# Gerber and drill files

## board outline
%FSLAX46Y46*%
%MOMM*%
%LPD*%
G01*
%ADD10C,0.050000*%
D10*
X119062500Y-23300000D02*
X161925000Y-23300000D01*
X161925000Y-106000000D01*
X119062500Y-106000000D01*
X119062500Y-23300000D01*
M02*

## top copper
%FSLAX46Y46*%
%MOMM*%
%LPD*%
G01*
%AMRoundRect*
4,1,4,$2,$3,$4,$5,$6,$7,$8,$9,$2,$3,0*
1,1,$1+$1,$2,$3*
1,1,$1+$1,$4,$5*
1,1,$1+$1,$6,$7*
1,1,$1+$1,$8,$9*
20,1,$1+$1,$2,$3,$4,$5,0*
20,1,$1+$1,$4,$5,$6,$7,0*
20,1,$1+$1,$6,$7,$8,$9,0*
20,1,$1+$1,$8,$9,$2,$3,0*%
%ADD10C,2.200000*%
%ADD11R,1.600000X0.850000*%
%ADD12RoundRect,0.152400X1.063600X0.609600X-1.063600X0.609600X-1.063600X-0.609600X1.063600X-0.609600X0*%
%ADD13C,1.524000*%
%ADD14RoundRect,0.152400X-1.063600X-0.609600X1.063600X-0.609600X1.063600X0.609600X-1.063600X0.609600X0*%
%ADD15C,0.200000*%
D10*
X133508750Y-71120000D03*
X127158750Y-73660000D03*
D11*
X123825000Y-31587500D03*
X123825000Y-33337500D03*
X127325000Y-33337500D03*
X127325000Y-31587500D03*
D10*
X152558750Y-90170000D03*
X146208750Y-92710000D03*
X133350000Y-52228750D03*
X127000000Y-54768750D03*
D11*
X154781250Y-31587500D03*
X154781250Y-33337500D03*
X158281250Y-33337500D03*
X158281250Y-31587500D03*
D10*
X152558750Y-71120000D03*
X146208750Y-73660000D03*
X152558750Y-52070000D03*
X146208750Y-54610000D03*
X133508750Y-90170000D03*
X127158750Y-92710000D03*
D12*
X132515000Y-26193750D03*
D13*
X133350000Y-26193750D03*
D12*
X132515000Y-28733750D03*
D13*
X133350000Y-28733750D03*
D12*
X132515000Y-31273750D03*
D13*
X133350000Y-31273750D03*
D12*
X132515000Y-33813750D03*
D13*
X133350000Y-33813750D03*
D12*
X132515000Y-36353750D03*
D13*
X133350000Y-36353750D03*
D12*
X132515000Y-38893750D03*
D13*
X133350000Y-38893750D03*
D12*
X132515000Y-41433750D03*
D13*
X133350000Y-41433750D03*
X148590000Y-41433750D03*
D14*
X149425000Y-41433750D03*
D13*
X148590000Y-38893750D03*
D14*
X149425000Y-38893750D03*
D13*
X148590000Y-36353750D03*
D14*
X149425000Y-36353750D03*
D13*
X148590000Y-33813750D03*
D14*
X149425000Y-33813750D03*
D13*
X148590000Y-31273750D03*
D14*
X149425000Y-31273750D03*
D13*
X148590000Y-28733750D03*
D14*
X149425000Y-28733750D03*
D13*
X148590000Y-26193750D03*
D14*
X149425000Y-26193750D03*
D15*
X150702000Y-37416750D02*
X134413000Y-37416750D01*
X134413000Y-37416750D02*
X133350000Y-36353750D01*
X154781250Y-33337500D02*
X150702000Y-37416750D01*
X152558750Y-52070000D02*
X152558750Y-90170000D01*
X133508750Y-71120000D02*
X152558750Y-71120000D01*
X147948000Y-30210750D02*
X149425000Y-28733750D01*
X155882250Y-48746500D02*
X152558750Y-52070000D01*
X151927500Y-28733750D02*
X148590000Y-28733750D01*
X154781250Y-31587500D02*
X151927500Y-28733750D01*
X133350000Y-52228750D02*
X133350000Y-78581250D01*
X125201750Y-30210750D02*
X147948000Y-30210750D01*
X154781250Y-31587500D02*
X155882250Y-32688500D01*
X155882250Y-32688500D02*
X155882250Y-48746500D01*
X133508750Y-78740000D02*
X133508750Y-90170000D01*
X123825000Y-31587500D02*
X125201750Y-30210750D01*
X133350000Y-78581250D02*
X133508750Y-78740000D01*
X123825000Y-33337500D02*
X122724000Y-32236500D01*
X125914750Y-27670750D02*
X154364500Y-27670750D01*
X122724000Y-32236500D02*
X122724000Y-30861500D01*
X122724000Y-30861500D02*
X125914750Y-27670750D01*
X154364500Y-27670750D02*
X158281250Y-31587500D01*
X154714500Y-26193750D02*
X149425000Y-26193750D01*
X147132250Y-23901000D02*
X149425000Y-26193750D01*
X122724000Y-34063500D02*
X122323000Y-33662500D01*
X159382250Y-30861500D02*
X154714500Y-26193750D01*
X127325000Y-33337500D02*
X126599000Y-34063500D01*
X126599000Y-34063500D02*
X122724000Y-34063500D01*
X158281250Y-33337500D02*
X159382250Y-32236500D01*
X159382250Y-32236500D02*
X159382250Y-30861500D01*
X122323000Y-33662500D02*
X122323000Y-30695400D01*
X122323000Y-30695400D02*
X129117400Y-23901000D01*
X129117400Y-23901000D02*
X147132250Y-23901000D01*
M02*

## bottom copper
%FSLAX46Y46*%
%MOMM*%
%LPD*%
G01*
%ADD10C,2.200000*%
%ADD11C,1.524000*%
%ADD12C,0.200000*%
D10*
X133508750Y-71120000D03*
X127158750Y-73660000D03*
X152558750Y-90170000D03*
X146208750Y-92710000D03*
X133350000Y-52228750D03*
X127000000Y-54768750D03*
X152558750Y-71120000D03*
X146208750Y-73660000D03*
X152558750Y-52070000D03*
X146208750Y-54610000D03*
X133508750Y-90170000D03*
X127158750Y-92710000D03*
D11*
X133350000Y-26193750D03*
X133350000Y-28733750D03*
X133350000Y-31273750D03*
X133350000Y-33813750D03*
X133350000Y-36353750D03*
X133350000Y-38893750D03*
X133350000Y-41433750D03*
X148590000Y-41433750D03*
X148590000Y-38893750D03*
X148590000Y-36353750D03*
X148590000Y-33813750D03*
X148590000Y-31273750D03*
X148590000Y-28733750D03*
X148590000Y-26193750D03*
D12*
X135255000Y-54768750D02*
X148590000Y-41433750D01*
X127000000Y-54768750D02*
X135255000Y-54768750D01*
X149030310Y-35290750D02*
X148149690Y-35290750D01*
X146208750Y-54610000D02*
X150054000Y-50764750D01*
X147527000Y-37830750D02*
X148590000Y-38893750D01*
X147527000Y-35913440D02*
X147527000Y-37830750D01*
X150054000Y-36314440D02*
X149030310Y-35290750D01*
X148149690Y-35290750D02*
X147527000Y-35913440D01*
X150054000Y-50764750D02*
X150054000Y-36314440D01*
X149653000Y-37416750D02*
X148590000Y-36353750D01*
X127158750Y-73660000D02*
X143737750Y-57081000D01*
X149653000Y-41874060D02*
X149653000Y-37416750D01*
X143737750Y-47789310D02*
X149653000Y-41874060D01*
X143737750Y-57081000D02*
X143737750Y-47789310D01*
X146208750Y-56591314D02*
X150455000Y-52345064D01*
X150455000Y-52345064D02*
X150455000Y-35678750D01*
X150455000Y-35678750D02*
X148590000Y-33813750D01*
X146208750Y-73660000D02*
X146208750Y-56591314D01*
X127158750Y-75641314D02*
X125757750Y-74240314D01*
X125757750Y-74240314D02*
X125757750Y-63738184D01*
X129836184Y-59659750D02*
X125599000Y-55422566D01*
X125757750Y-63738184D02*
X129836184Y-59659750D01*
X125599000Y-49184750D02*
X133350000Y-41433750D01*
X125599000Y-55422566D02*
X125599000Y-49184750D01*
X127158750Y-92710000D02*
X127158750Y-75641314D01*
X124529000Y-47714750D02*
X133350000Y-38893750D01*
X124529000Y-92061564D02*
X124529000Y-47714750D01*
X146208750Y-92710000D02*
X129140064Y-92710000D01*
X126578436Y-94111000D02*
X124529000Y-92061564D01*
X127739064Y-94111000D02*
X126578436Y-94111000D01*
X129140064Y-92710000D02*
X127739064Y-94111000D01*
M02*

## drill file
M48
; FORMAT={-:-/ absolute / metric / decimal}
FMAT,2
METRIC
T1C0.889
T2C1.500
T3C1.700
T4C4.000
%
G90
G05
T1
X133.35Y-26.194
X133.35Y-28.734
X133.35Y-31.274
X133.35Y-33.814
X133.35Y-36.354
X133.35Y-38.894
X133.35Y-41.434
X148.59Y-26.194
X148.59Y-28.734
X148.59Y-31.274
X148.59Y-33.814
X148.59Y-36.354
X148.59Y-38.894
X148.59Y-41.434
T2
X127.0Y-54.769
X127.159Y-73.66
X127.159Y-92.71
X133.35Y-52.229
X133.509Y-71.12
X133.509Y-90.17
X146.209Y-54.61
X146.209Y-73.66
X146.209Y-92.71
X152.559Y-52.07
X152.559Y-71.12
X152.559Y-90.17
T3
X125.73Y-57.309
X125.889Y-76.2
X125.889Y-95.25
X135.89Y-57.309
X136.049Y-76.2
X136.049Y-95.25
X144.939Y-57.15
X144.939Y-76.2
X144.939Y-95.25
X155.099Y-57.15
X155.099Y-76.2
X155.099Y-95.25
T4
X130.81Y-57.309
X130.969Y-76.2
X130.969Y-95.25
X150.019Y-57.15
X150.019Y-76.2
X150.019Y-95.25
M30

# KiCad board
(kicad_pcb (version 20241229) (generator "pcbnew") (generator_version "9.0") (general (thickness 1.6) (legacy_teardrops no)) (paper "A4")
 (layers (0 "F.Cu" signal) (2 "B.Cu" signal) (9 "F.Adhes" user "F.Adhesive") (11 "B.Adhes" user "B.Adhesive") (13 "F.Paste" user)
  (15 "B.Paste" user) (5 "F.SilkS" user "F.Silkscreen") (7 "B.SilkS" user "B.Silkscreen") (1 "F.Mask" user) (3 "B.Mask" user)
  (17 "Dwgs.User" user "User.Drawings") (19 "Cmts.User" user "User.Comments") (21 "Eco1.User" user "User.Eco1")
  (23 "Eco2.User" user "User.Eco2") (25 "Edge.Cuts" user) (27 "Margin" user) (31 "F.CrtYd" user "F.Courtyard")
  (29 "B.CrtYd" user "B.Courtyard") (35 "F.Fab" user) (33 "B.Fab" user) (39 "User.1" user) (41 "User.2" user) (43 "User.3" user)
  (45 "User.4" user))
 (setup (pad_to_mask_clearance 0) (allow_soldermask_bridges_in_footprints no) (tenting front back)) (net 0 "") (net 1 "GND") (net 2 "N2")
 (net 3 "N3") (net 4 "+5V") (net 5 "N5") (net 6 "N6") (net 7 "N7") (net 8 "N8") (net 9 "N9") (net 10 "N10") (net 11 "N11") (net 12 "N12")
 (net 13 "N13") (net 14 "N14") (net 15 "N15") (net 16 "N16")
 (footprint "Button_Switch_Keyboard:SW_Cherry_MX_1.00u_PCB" (layer "F.Cu") (at 133.50875 71.12)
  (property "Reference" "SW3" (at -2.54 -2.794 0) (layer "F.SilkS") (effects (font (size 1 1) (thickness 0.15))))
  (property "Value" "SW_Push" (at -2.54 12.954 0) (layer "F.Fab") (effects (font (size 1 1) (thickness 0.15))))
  (pad "" np_thru_hole circle (at -7.62 5.08) (size 1.7 1.7) (drill 1.7) (layers "*.Cu" "*.Mask"))
  (pad "" np_thru_hole circle (at -2.54 5.08) (size 4 4) (drill 4) (layers "*.Cu" "*.Mask"))
  (pad "" np_thru_hole circle (at 2.54 5.08) (size 1.7 1.7) (drill 1.7) (layers "*.Cu" "*.Mask"))
  (pad "1" thru_hole circle (at 0 0) (size 2.2 2.2) (drill 1.5) (layers "*.Cu" "*.Mask") (remove_unused_layers no) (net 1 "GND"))
  (pad "2" thru_hole circle (at -6.35 2.54) (size 2.2 2.2) (drill 1.5) (layers "*.Cu" "*.Mask") (remove_unused_layers no) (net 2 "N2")))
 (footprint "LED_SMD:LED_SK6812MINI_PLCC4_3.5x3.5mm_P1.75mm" (layer "F.Cu") (at 125.575 32.4625)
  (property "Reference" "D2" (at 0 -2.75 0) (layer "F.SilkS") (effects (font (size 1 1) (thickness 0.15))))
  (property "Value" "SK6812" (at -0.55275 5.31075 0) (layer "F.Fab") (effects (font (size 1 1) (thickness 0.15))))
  (pad "1" smd rect (at -1.75 -0.875) (size 1.6 0.85) (layers "F.Cu" "F.Mask" "F.Paste") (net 1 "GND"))
  (pad "2" smd rect (at -1.75 0.875) (size 1.6 0.85) (layers "F.Cu" "F.Mask" "F.Paste") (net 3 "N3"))
  (pad "3" smd rect (at 1.75 0.875) (size 1.6 0.85) (layers "F.Cu" "F.Mask" "F.Paste") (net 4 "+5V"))
  (pad "4" smd rect (at 1.75 -0.875) (size 1.6 0.85) (layers "F.Cu" "F.Mask" "F.Paste") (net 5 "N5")))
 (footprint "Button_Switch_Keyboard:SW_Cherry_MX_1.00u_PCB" (layer "F.Cu") (at 152.55875 90.17)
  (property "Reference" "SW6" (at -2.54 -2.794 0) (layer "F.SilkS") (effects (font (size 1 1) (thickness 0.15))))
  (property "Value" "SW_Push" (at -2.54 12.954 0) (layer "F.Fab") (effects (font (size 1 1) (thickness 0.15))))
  (pad "" np_thru_hole circle (at -7.62 5.08) (size 1.7 1.7) (drill 1.7) (layers "*.Cu" "*.Mask"))
  (pad "" np_thru_hole circle (at -2.54 5.08) (size 4 4) (drill 4) (layers "*.Cu" "*.Mask"))
  (pad "" np_thru_hole circle (at 2.54 5.08) (size 1.7 1.7) (drill 1.7) (layers "*.Cu" "*.Mask"))
  (pad "1" thru_hole circle (at 0 0) (size 2.2 2.2) (drill 1.5) (layers "*.Cu" "*.Mask") (remove_unused_layers no) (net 1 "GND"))
  (pad "2" thru_hole circle (at -6.35 2.54) (size 2.2 2.2) (drill 1.5) (layers "*.Cu" "*.Mask") (remove_unused_layers no) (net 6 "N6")))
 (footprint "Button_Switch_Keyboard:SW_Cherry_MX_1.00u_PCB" (layer "F.Cu") (at 133.35 52.22875)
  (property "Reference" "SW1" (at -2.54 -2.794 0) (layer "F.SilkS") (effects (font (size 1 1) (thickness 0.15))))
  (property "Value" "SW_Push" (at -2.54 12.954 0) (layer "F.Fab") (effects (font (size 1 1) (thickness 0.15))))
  (pad "" np_thru_hole circle (at -7.62 5.08) (size 1.7 1.7) (drill 1.7) (layers "*.Cu" "*.Mask"))
  (pad "" np_thru_hole circle (at -2.54 5.08) (size 4 4) (drill 4) (layers "*.Cu" "*.Mask"))
  (pad "" np_thru_hole circle (at 2.54 5.08) (size 1.7 1.7) (drill 1.7) (layers "*.Cu" "*.Mask"))
  (pad "1" thru_hole circle (at 0 0) (size 2.2 2.2) (drill 1.5) (layers "*.Cu" "*.Mask") (remove_unused_layers no) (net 1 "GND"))
  (pad "2" thru_hole circle (at -6.35 2.54) (size 2.2 2.2) (drill 1.5) (layers "*.Cu" "*.Mask") (remove_unused_layers no) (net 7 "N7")))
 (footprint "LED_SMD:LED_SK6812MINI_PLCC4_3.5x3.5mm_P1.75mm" (layer "F.Cu") (at 156.53125 32.4625)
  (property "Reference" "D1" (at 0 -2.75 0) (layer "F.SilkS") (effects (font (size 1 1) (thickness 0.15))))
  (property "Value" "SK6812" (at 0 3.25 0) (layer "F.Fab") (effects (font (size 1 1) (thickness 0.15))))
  (pad "1" smd rect (at -1.75 -0.875) (size 1.6 0.85) (layers "F.Cu" "F.Mask" "F.Paste") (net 1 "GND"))
  (pad "2" smd rect (at -1.75 0.875) (size 1.6 0.85) (layers "F.Cu" "F.Mask" "F.Paste") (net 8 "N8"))
  (pad "3" smd rect (at 1.75 0.875) (size 1.6 0.85) (layers "F.Cu" "F.Mask" "F.Paste") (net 4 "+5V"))
  (pad "4" smd rect (at 1.75 -0.875) (size 1.6 0.85) (layers "F.Cu" "F.Mask" "F.Paste") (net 3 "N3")))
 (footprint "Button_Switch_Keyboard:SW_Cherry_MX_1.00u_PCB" (layer "F.Cu") (at 152.55875 71.12)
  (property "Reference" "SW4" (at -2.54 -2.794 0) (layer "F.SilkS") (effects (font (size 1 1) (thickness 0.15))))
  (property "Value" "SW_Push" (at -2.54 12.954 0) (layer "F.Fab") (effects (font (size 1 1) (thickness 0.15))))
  (pad "" np_thru_hole circle (at -7.62 5.08) (size 1.7 1.7) (drill 1.7) (layers "*.Cu" "*.Mask"))
  (pad "" np_thru_hole circle (at -2.54 5.08) (size 4 4) (drill 4) (layers "*.Cu" "*.Mask"))
  (pad "" np_thru_hole circle (at 2.54 5.08) (size 1.7 1.7) (drill 1.7) (layers "*.Cu" "*.Mask"))
  (pad "1" thru_hole circle (at 0 0) (size 2.2 2.2) (drill 1.5) (layers "*.Cu" "*.Mask") (remove_unused_layers no) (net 1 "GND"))
  (pad "2" thru_hole circle (at -6.35 2.54) (size 2.2 2.2) (drill 1.5) (layers "*.Cu" "*.Mask") (remove_unused_layers no) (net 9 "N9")))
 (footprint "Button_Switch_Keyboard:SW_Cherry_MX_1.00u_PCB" (layer "F.Cu") (at 152.55875 52.07)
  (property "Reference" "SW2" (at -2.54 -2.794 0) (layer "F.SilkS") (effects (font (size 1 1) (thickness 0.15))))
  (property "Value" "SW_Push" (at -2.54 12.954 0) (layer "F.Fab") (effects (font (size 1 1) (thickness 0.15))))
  (pad "" np_thru_hole circle (at -7.62 5.08) (size 1.7 1.7) (drill 1.7) (layers "*.Cu" "*.Mask"))
  (pad "" np_thru_hole circle (at -2.54 5.08) (size 4 4) (drill 4) (layers "*.Cu" "*.Mask"))
  (pad "" np_thru_hole circle (at 2.54 5.08) (size 1.7 1.7) (drill 1.7) (layers "*.Cu" "*.Mask"))
  (pad "1" thru_hole circle (at 0 0) (size 2.2 2.2) (drill 1.5) (layers "*.Cu" "*.Mask") (remove_unused_layers no) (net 1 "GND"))
  (pad "2" thru_hole circle (at -6.35 2.54) (size 2.2 2.2) (drill 1.5) (layers "*.Cu" "*.Mask") (remove_unused_layers no) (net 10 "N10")))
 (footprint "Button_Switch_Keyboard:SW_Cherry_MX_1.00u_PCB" (layer "F.Cu") (at 133.50875 90.17)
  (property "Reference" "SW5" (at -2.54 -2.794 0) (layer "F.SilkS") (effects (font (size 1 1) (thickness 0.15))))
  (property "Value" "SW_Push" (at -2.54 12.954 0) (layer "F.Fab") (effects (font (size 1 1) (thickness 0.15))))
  (pad "" np_thru_hole circle (at -7.62 5.08) (size 1.7 1.7) (drill 1.7) (layers "*.Cu" "*.Mask"))
  (pad "" np_thru_hole circle (at -2.54 5.08) (size 4 4) (drill 4) (layers "*.Cu" "*.Mask"))
  (pad "" np_thru_hole circle (at 2.54 5.08) (size 1.7 1.7) (drill 1.7) (layers "*.Cu" "*.Mask"))
  (pad "1" thru_hole circle (at 0 0) (size 2.2 2.2) (drill 1.5) (layers "*.Cu" "*.Mask") (remove_unused_layers no) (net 1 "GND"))
  (pad "2" thru_hole circle (at -6.35 2.54) (size 2.2 2.2) (drill 1.5) (layers "*.Cu" "*.Mask") (remove_unused_layers no) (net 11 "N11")))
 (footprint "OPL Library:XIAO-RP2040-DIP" (layer "F.Cu") (at 140.97 33.81375)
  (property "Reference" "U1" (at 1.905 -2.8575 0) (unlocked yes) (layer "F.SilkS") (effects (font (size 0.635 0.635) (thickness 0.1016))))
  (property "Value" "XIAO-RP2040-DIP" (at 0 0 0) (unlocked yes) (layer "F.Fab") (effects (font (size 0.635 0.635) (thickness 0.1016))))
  (pad "1" smd roundrect (at -8.455 -7.62 180) (size 2.432 1.524) (layers "F.Cu" "F.Mask") (roundrect_rratio 0.1) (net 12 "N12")
   (thermal_bridge_angle 45))
  (pad "1" thru_hole circle (at -7.62 -7.62 180) (size 1.524 1.524) (drill 0.889) (layers "*.Cu" "*.Mask") (remove_unused_layers no)
   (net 12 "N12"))
  (pad "2" smd roundrect (at -8.455 -5.08 180) (size 2.432 1.524) (layers "F.Cu" "F.Mask") (roundrect_rratio 0.1) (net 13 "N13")
   (thermal_bridge_angle 45))
  (pad "2" thru_hole circle (at -7.62 -5.08 180) (size 1.524 1.524) (drill 0.889) (layers "*.Cu" "*.Mask") (remove_unused_layers no)
   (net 13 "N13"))
  (pad "3" smd roundrect (at -8.455 -2.54 180) (size 2.432 1.524) (layers "F.Cu" "F.Mask") (roundrect_rratio 0.1) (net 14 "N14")
   (thermal_bridge_angle 45))
  (pad "3" thru_hole circle (at -7.62 -2.54 180) (size 1.524 1.524) (drill 0.889) (layers "*.Cu" "*.Mask") (remove_unused_layers no)
   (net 14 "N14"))
  (pad "4" smd roundrect (at -8.455 0 180) (size 2.432 1.524) (layers "F.Cu" "F.Mask") (roundrect_rratio 0.1) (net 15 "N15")
   (thermal_bridge_angle 45))
  (pad "4" thru_hole circle (at -7.62 0 180) (size 1.524 1.524) (drill 0.889) (layers "*.Cu" "*.Mask") (remove_unused_layers no)
   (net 15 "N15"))
  (pad "5" smd roundrect (at -8.455 2.54 180) (size 2.432 1.524) (layers "F.Cu" "F.Mask") (roundrect_rratio 0.1) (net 8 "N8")
   (thermal_bridge_angle 45))
  (pad "5" thru_hole circle (at -7.62 2.54 180) (size 1.524 1.524) (drill 0.889) (layers "*.Cu" "*.Mask") (remove_unused_layers no)
   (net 8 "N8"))
  (pad "6" smd roundrect (at -8.455 5.08 180) (size 2.432 1.524) (layers "F.Cu" "F.Mask") (roundrect_rratio 0.1) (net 6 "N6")
   (thermal_bridge_angle 45))
  (pad "6" thru_hole circle (at -7.62 5.08 180) (size 1.524 1.524) (drill 0.889) (layers "*.Cu" "*.Mask") (remove_unused_layers no)
   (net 6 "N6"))
  (pad "7" smd roundrect (at -8.455 7.62 180) (size 2.432 1.524) (layers "F.Cu" "F.Mask") (roundrect_rratio 0.1) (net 11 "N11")
   (thermal_bridge_angle 45))
  (pad "7" thru_hole circle (at -7.62 7.62 180) (size 1.524 1.524) (drill 0.889) (layers "*.Cu" "*.Mask") (remove_unused_layers no)
   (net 11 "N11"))
  (pad "8" thru_hole circle (at 7.62 7.62) (size 1.524 1.524) (drill 0.889) (layers "*.Cu" "*.Mask") (remove_unused_layers no) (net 7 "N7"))
  (pad "8" smd roundrect (at 8.455 7.62) (size 2.432 1.524) (layers "F.Cu" "F.Mask") (roundrect_rratio 0.1) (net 7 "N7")
   (thermal_bridge_angle 45))
  (pad "9" thru_hole circle (at 7.62 5.08) (size 1.524 1.524) (drill 0.889) (layers "*.Cu" "*.Mask") (remove_unused_layers no)
   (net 10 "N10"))
  (pad "9" smd roundrect (at 8.455 5.08) (size 2.432 1.524) (layers "F.Cu" "F.Mask") (roundrect_rratio 0.1) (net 10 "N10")
   (thermal_bridge_angle 45))
  (pad "10" thru_hole circle (at 7.62 2.54) (size 1.524 1.524) (drill 0.889) (layers "*.Cu" "*.Mask") (remove_unused_layers no) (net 2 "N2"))
  (pad "10" smd roundrect (at 8.455 2.54) (size 2.432 1.524) (layers "F.Cu" "F.Mask") (roundrect_rratio 0.1) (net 2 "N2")
   (thermal_bridge_angle 45))
  (pad "11" thru_hole circle (at 7.62 0) (size 1.524 1.524) (drill 0.889) (layers "*.Cu" "*.Mask") (remove_unused_layers no) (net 9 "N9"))
  (pad "11" smd roundrect (at 8.455 0) (size 2.432 1.524) (layers "F.Cu" "F.Mask") (roundrect_rratio 0.1) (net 9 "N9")
   (thermal_bridge_angle 45))
  (pad "12" thru_hole circle (at 7.62 -2.54) (size 1.524 1.524) (drill 0.889) (layers "*.Cu" "*.Mask") (remove_unused_layers no)
   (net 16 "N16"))
  (pad "12" smd roundrect (at 8.455 -2.54) (size 2.432 1.524) (layers "F.Cu" "F.Mask") (roundrect_rratio 0.1) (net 16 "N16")
   (thermal_bridge_angle 45))
  (pad "13" thru_hole circle (at 7.62 -5.08) (size 1.524 1.524) (drill 0.889) (layers "*.Cu" "*.Mask") (remove_unused_layers no)
   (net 1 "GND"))
  (pad "13" smd roundrect (at 8.455 -5.08) (size 2.432 1.524) (layers "F.Cu" "F.Mask") (roundrect_rratio 0.1) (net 1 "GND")
   (thermal_bridge_angle 45))
  (pad "14" thru_hole circle (at 7.62 -7.62) (size 1.524 1.524) (drill 0.889) (layers "*.Cu" "*.Mask") (remove_unused_layers no)
   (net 4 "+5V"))
  (pad "14" smd roundrect (at 8.455 -7.62) (size 2.432 1.524) (layers "F.Cu" "F.Mask") (roundrect_rratio 0.1) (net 4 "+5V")
   (thermal_bridge_angle 45)))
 (gr_rect (start 119.0625 23.3) (end 161.925 106) (stroke (width 0.05) (type solid)) (fill no) (layer "Edge.Cuts"))
 (segment (start 150.702 37.41675) (end 134.413 37.41675) (width 0.2) (layer "F.Cu") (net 8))
 (segment (start 134.413 37.41675) (end 133.35 36.35375) (width 0.2) (layer "F.Cu") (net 8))
 (segment (start 154.78125 33.3375) (end 150.702 37.41675) (width 0.2) (layer "F.Cu") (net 8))
 (segment (start 152.55875 52.07) (end 152.55875 90.17) (width 0.2) (layer "F.Cu") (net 1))
 (segment (start 133.50875 71.12) (end 152.55875 71.12) (width 0.2) (layer "F.Cu") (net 1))
 (segment (start 147.948 30.21075) (end 149.425 28.73375) (width 0.2) (layer "F.Cu") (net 1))
 (segment (start 155.88225 48.7465) (end 152.55875 52.07) (width 0.2) (layer "F.Cu") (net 1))
 (segment (start 151.9275 28.73375) (end 148.59 28.73375) (width 0.2) (layer "F.Cu") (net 1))
 (segment (start 154.78125 31.5875) (end 151.9275 28.73375) (width 0.2) (layer "F.Cu") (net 1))
 (segment (start 133.35 52.22875) (end 133.35 78.58125) (width 0.2) (layer "F.Cu") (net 1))
 (segment (start 125.20175 30.21075) (end 147.948 30.21075) (width 0.2) (layer "F.Cu") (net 1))
 (segment (start 154.78125 31.5875) (end 155.88225 32.6885) (width 0.2) (layer "F.Cu") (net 1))
 (segment (start 155.88225 32.6885) (end 155.88225 48.7465) (width 0.2) (layer "F.Cu") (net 1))
 (segment (start 133.50875 78.74) (end 133.50875 90.17) (width 0.2) (layer "F.Cu") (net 1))
 (segment (start 123.825 31.5875) (end 125.20175 30.21075) (width 0.2) (layer "F.Cu") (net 1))
 (segment (start 133.35 78.58125) (end 133.50875 78.74) (width 0.2) (layer "F.Cu") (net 1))
 (segment (start 123.825 33.3375) (end 122.724 32.2365) (width 0.2) (layer "F.Cu") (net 3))
 (segment (start 125.91475 27.67075) (end 154.3645 27.67075) (width 0.2) (layer "F.Cu") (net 3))
 (segment (start 122.724 32.2365) (end 122.724 30.8615) (width 0.2) (layer "F.Cu") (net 3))
 (segment (start 122.724 30.8615) (end 125.91475 27.67075) (width 0.2) (layer "F.Cu") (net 3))
 (segment (start 154.3645 27.67075) (end 158.28125 31.5875) (width 0.2) (layer "F.Cu") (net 3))
 (segment (start 154.7145 26.19375) (end 149.425 26.19375) (width 0.2) (layer "F.Cu") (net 4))
 (segment (start 147.13225 23.901) (end 149.425 26.19375) (width 0.2) (layer "F.Cu") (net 4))
 (segment (start 122.724 34.0635) (end 122.323 33.6625) (width 0.2) (layer "F.Cu") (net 4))
 (segment (start 159.38225 30.8615) (end 154.7145 26.19375) (width 0.2) (layer "F.Cu") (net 4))
 (segment (start 127.325 33.3375) (end 126.599 34.0635) (width 0.2) (layer "F.Cu") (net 4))
 (segment (start 126.599 34.0635) (end 122.724 34.0635) (width 0.2) (layer "F.Cu") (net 4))
 (segment (start 158.28125 33.3375) (end 159.38225 32.2365) (width 0.2) (layer "F.Cu") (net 4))
 (segment (start 159.38225 32.2365) (end 159.38225 30.8615) (width 0.2) (layer "F.Cu") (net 4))
 (segment (start 122.323 33.6625) (end 122.323 30.6954) (width 0.2) (layer "F.Cu") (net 4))
 (segment (start 122.323 30.6954) (end 129.1174 23.901) (width 0.2) (layer "F.Cu") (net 4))
 (segment (start 129.1174 23.901) (end 147.13225 23.901) (width 0.2) (layer "F.Cu") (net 4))
 (segment (start 135.255 54.76875) (end 148.59 41.43375) (width 0.2) (layer "B.Cu") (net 7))
 (segment (start 127 54.76875) (end 135.255 54.76875) (width 0.2) (layer "B.Cu") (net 7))
 (segment (start 149.03031 35.29075) (end 148.14969 35.29075) (width 0.2) (layer "B.Cu") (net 10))
 (segment (start 146.20875 54.61) (end 150.054 50.76475) (width 0.2) (layer "B.Cu") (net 10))
 (segment (start 147.527 37.83075) (end 148.59 38.89375) (width 0.2) (layer "B.Cu") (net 10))
 (segment (start 147.527 35.91344) (end 147.527 37.83075) (width 0.2) (layer "B.Cu") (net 10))
 (segment (start 150.054 36.31444) (end 149.03031 35.29075) (width 0.2) (layer "B.Cu") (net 10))
 (segment (start 148.14969 35.29075) (end 147.527 35.91344) (width 0.2) (layer "B.Cu") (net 10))
 (segment (start 150.054 50.76475) (end 150.054 36.31444) (width 0.2) (layer "B.Cu") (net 10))
 (segment (start 149.653 37.41675) (end 148.59 36.35375) (width 0.2) (layer "B.Cu") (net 2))
 (segment (start 127.15875 73.66) (end 143.73775 57.081) (width 0.2) (layer "B.Cu") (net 2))
 (segment (start 149.653 41.87406) (end 149.653 37.41675) (width 0.2) (layer "B.Cu") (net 2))
 (segment (start 143.73775 47.78931) (end 149.653 41.87406) (width 0.2) (layer "B.Cu") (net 2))
 (segment (start 143.73775 57.081) (end 143.73775 47.78931) (width 0.2) (layer "B.Cu") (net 2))
 (segment (start 146.20875 56.591314) (end 150.455 52.345064) (width 0.2) (layer "B.Cu") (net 9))
 (segment (start 150.455 52.345064) (end 150.455 35.67875) (width 0.2) (layer "B.Cu") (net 9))
 (segment (start 150.455 35.67875) (end 148.59 33.81375) (width 0.2) (layer "B.Cu") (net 9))
 (segment (start 146.20875 73.66) (end 146.20875 56.591314) (width 0.2) (layer "B.Cu") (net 9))
 (segment (start 127.15875 75.641314) (end 125.75775 74.240314) (width 0.2) (layer "B.Cu") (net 11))
 (segment (start 125.75775 74.240314) (end 125.75775 63.738184) (width 0.2) (layer "B.Cu") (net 11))
 (segment (start 129.836184 59.65975) (end 125.599 55.422566) (width 0.2) (layer "B.Cu") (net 11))
 (segment (start 125.75775 63.738184) (end 129.836184 59.65975) (width 0.2) (layer "B.Cu") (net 11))
 (segment (start 125.599 49.18475) (end 133.35 41.43375) (width 0.2) (layer "B.Cu") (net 11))
 (segment (start 125.599 55.422566) (end 125.599 49.18475) (width 0.2) (layer "B.Cu") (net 11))
 (segment (start 127.15875 92.71) (end 127.15875 75.641314) (width 0.2) (layer "B.Cu") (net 11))
 (segment (start 124.529 47.71475) (end 133.35 38.89375) (width 0.2) (layer "B.Cu") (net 6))
 (segment (start 124.529 92.061564) (end 124.529 47.71475) (width 0.2) (layer "B.Cu") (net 6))
 (segment (start 146.20875 92.71) (end 129.140064 92.71) (width 0.2) (layer "B.Cu") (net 6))
 (segment (start 126.578436 94.111) (end 124.529 92.061564) (width 0.2) (layer "B.Cu") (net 6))
 (segment (start 127.739064 94.111) (end 126.578436 94.111) (width 0.2) (layer "B.Cu") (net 6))
 (segment (start 129.140064 92.71) (end 127.739064 94.111) (width 0.2) (layer "B.Cu") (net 6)))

